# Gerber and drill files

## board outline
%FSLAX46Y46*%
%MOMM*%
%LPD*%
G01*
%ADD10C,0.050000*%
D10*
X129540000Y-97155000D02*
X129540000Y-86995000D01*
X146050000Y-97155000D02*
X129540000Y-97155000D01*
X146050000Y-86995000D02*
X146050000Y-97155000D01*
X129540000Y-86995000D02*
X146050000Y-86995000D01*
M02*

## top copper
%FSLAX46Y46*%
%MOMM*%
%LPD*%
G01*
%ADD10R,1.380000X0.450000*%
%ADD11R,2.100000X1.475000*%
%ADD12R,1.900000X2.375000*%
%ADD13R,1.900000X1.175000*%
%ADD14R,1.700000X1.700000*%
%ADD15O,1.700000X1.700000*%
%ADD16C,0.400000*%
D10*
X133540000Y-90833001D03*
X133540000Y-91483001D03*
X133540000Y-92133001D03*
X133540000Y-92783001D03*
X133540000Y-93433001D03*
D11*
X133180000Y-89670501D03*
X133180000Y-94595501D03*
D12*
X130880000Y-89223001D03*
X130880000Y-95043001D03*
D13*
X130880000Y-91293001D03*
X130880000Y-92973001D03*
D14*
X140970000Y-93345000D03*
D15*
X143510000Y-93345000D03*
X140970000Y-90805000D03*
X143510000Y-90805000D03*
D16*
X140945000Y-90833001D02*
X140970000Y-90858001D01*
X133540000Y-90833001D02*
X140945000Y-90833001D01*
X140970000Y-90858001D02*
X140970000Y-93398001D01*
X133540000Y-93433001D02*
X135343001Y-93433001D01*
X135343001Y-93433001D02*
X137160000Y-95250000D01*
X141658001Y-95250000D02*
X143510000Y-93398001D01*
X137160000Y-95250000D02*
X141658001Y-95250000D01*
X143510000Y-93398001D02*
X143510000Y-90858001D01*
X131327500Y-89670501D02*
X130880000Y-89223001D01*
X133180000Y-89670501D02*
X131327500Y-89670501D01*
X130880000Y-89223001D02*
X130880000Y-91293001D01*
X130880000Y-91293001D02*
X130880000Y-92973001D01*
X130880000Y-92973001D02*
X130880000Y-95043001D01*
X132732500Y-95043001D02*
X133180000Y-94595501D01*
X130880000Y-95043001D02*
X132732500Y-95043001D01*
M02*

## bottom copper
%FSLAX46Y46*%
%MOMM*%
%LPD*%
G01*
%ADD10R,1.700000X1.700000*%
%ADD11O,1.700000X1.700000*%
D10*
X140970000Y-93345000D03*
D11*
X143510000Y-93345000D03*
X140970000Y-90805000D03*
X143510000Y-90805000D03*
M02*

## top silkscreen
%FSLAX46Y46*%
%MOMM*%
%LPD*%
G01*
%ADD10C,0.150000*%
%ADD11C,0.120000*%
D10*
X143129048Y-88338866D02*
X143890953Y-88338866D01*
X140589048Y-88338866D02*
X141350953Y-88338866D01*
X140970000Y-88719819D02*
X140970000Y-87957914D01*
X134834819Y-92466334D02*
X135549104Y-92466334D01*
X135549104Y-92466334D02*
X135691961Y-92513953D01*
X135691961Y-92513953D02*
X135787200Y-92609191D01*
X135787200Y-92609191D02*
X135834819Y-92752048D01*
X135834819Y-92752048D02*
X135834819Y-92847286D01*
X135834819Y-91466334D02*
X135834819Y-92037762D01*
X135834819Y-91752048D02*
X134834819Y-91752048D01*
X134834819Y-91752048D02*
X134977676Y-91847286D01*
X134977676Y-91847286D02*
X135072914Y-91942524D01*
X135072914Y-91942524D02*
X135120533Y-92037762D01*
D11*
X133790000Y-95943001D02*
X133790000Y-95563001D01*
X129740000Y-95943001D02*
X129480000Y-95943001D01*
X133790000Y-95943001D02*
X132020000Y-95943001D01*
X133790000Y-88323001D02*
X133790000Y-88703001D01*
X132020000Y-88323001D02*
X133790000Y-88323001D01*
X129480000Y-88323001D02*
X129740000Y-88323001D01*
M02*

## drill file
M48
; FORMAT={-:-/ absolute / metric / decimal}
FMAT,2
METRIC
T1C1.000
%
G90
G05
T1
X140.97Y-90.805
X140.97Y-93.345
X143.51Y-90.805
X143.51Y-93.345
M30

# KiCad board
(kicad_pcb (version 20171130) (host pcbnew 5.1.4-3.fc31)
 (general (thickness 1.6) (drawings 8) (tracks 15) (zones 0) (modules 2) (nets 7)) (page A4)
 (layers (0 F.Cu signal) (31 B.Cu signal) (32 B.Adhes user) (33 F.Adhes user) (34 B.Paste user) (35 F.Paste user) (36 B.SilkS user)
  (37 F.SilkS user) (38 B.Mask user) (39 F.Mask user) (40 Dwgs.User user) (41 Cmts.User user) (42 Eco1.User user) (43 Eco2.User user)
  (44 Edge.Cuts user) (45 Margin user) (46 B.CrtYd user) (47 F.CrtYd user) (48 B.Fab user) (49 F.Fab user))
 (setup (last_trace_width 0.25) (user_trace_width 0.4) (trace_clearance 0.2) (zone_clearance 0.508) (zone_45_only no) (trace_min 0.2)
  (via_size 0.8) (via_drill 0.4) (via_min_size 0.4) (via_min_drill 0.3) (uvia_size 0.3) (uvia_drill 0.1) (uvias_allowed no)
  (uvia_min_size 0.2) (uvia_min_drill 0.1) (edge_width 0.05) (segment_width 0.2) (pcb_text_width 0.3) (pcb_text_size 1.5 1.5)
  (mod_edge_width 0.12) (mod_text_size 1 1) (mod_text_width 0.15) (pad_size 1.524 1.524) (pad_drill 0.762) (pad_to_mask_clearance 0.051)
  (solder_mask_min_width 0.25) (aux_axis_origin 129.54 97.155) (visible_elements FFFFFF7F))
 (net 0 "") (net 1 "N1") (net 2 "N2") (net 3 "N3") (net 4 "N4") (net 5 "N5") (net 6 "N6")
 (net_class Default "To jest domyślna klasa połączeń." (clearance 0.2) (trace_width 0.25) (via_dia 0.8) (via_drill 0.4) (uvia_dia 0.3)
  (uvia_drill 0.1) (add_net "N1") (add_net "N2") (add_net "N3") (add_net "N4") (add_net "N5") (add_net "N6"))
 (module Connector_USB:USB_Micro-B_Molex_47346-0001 (layer F.Cu) (at 132.08 92.133001 270)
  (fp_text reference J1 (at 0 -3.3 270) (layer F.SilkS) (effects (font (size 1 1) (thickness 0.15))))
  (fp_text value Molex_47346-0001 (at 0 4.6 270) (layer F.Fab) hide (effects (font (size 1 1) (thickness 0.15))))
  (fp_line (start 3.81 -1.71) (end 3.43 -1.71) (layer F.SilkS) (width 0.12))
  (fp_line (start 3.81 2.34) (end 3.81 2.6) (layer F.SilkS) (width 0.12))
  (fp_line (start 3.81 -1.71) (end 3.81 0.06) (layer F.SilkS) (width 0.12))
  (fp_line (start -3.81 -1.71) (end -3.43 -1.71) (layer F.SilkS) (width 0.12))
  (fp_line (start -3.81 0.06) (end -3.81 -1.71) (layer F.SilkS) (width 0.12))
  (fp_line (start -3.81 2.6) (end -3.81 2.34) (layer F.SilkS) (width 0.12))
  (pad 1 smd rect (at -1.3 -1.46 270) (size 0.45 1.38) (layers F.Cu F.Paste F.Mask) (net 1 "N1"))
  (pad 2 smd rect (at -0.65 -1.46 270) (size 0.45 1.38) (layers F.Cu F.Paste F.Mask) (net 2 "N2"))
  (pad 3 smd rect (at 0 -1.46 270) (size 0.45 1.38) (layers F.Cu F.Paste F.Mask) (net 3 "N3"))
  (pad 4 smd rect (at 0.65 -1.46 270) (size 0.45 1.38) (layers F.Cu F.Paste F.Mask) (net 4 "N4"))
  (pad 5 smd rect (at 1.3 -1.46 270) (size 0.45 1.38) (layers F.Cu F.Paste F.Mask) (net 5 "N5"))
  (pad 6 smd rect (at -2.4625 -1.1 270) (size 1.475 2.1) (layers F.Cu F.Paste F.Mask) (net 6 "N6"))
  (pad 6 smd rect (at 2.4625 -1.1 270) (size 1.475 2.1) (layers F.Cu F.Paste F.Mask) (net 6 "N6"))
  (pad 6 smd rect (at -2.91 1.2 270) (size 2.375 1.9) (layers F.Cu F.Paste F.Mask) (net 6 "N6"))
  (pad 6 smd rect (at 2.91 1.2 270) (size 2.375 1.9) (layers F.Cu F.Paste F.Mask) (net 6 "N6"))
  (pad 6 smd rect (at -0.84 1.2 270) (size 1.175 1.9) (layers F.Cu F.Paste F.Mask) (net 6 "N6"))
  (pad 6 smd rect (at 0.84 1.2 270) (size 1.175 1.9) (layers F.Cu F.Paste F.Mask) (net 6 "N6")))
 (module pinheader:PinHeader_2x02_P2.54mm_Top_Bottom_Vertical (layer B.Cu) (at 140.97 93.345)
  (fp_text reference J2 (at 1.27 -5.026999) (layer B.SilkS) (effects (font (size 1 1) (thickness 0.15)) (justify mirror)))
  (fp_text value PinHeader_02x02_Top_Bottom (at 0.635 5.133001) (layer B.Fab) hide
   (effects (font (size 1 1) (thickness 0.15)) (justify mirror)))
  (pad 1 thru_hole rect (at 0 0) (size 1.7 1.7) (drill 1) (layers *.Cu *.Mask) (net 1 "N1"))
  (pad 3 thru_hole oval (at 2.54 0) (size 1.7 1.7) (drill 1) (layers *.Cu *.Mask) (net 5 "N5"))
  (pad 2 thru_hole oval (at 0 -2.54) (size 1.7 1.7) (drill 1) (layers *.Cu *.Mask) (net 1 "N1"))
  (pad 4 thru_hole oval (at 2.54 -2.54) (size 1.7 1.7) (drill 1) (layers *.Cu *.Mask) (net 5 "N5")))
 (gr_line (start 129.54 97.155) (end 129.54 86.995) (layer Edge.Cuts) (width 0.05))
 (gr_line (start 146.05 97.155) (end 129.54 97.155) (layer Edge.Cuts) (width 0.05))
 (gr_line (start 146.05 86.995) (end 146.05 97.155) (layer Edge.Cuts) (width 0.05))
 (gr_line (start 129.54 86.995) (end 146.05 86.995) (layer Edge.Cuts) (width 0.05))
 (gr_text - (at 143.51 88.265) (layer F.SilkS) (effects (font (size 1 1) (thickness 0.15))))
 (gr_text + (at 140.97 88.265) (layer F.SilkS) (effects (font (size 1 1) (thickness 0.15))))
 (segment (start 140.945 90.833001) (end 140.97 90.858001) (width 0.4) (layer F.Cu) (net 1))
 (segment (start 133.54 90.833001) (end 140.945 90.833001) (width 0.4) (layer F.Cu) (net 1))
 (segment (start 140.97 90.858001) (end 140.97 93.398001) (width 0.4) (layer F.Cu) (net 1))
 (segment (start 133.54 93.433001) (end 135.343001 93.433001) (width 0.4) (layer F.Cu) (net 5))
 (segment (start 135.343001 93.433001) (end 137.16 95.25) (width 0.4) (layer F.Cu) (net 5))
 (segment (start 141.658001 95.25) (end 143.51 93.398001) (width 0.4) (layer F.Cu) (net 5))
 (segment (start 137.16 95.25) (end 141.658001 95.25) (width 0.4) (layer F.Cu) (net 5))
 (segment (start 143.51 93.398001) (end 143.51 90.858001) (width 0.4) (layer F.Cu) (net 5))
 (segment (start 131.3275 89.670501) (end 130.88 89.223001) (width 0.4) (layer F.Cu) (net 6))
 (segment (start 133.18 89.670501) (end 131.3275 89.670501) (width 0.4) (layer F.Cu) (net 6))
 (segment (start 130.88 89.223001) (end 130.88 91.293001) (width 0.4) (layer F.Cu) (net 6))
 (segment (start 130.88 91.293001) (end 130.88 92.973001) (width 0.4) (layer F.Cu) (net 6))
 (segment (start 130.88 92.973001) (end 130.88 95.043001) (width 0.4) (layer F.Cu) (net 6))
 (segment (start 132.7325 95.043001) (end 133.18 94.595501) (width 0.4) (layer F.Cu) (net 6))
 (segment (start 130.88 95.043001) (end 132.7325 95.043001) (width 0.4) (layer F.Cu) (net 6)))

